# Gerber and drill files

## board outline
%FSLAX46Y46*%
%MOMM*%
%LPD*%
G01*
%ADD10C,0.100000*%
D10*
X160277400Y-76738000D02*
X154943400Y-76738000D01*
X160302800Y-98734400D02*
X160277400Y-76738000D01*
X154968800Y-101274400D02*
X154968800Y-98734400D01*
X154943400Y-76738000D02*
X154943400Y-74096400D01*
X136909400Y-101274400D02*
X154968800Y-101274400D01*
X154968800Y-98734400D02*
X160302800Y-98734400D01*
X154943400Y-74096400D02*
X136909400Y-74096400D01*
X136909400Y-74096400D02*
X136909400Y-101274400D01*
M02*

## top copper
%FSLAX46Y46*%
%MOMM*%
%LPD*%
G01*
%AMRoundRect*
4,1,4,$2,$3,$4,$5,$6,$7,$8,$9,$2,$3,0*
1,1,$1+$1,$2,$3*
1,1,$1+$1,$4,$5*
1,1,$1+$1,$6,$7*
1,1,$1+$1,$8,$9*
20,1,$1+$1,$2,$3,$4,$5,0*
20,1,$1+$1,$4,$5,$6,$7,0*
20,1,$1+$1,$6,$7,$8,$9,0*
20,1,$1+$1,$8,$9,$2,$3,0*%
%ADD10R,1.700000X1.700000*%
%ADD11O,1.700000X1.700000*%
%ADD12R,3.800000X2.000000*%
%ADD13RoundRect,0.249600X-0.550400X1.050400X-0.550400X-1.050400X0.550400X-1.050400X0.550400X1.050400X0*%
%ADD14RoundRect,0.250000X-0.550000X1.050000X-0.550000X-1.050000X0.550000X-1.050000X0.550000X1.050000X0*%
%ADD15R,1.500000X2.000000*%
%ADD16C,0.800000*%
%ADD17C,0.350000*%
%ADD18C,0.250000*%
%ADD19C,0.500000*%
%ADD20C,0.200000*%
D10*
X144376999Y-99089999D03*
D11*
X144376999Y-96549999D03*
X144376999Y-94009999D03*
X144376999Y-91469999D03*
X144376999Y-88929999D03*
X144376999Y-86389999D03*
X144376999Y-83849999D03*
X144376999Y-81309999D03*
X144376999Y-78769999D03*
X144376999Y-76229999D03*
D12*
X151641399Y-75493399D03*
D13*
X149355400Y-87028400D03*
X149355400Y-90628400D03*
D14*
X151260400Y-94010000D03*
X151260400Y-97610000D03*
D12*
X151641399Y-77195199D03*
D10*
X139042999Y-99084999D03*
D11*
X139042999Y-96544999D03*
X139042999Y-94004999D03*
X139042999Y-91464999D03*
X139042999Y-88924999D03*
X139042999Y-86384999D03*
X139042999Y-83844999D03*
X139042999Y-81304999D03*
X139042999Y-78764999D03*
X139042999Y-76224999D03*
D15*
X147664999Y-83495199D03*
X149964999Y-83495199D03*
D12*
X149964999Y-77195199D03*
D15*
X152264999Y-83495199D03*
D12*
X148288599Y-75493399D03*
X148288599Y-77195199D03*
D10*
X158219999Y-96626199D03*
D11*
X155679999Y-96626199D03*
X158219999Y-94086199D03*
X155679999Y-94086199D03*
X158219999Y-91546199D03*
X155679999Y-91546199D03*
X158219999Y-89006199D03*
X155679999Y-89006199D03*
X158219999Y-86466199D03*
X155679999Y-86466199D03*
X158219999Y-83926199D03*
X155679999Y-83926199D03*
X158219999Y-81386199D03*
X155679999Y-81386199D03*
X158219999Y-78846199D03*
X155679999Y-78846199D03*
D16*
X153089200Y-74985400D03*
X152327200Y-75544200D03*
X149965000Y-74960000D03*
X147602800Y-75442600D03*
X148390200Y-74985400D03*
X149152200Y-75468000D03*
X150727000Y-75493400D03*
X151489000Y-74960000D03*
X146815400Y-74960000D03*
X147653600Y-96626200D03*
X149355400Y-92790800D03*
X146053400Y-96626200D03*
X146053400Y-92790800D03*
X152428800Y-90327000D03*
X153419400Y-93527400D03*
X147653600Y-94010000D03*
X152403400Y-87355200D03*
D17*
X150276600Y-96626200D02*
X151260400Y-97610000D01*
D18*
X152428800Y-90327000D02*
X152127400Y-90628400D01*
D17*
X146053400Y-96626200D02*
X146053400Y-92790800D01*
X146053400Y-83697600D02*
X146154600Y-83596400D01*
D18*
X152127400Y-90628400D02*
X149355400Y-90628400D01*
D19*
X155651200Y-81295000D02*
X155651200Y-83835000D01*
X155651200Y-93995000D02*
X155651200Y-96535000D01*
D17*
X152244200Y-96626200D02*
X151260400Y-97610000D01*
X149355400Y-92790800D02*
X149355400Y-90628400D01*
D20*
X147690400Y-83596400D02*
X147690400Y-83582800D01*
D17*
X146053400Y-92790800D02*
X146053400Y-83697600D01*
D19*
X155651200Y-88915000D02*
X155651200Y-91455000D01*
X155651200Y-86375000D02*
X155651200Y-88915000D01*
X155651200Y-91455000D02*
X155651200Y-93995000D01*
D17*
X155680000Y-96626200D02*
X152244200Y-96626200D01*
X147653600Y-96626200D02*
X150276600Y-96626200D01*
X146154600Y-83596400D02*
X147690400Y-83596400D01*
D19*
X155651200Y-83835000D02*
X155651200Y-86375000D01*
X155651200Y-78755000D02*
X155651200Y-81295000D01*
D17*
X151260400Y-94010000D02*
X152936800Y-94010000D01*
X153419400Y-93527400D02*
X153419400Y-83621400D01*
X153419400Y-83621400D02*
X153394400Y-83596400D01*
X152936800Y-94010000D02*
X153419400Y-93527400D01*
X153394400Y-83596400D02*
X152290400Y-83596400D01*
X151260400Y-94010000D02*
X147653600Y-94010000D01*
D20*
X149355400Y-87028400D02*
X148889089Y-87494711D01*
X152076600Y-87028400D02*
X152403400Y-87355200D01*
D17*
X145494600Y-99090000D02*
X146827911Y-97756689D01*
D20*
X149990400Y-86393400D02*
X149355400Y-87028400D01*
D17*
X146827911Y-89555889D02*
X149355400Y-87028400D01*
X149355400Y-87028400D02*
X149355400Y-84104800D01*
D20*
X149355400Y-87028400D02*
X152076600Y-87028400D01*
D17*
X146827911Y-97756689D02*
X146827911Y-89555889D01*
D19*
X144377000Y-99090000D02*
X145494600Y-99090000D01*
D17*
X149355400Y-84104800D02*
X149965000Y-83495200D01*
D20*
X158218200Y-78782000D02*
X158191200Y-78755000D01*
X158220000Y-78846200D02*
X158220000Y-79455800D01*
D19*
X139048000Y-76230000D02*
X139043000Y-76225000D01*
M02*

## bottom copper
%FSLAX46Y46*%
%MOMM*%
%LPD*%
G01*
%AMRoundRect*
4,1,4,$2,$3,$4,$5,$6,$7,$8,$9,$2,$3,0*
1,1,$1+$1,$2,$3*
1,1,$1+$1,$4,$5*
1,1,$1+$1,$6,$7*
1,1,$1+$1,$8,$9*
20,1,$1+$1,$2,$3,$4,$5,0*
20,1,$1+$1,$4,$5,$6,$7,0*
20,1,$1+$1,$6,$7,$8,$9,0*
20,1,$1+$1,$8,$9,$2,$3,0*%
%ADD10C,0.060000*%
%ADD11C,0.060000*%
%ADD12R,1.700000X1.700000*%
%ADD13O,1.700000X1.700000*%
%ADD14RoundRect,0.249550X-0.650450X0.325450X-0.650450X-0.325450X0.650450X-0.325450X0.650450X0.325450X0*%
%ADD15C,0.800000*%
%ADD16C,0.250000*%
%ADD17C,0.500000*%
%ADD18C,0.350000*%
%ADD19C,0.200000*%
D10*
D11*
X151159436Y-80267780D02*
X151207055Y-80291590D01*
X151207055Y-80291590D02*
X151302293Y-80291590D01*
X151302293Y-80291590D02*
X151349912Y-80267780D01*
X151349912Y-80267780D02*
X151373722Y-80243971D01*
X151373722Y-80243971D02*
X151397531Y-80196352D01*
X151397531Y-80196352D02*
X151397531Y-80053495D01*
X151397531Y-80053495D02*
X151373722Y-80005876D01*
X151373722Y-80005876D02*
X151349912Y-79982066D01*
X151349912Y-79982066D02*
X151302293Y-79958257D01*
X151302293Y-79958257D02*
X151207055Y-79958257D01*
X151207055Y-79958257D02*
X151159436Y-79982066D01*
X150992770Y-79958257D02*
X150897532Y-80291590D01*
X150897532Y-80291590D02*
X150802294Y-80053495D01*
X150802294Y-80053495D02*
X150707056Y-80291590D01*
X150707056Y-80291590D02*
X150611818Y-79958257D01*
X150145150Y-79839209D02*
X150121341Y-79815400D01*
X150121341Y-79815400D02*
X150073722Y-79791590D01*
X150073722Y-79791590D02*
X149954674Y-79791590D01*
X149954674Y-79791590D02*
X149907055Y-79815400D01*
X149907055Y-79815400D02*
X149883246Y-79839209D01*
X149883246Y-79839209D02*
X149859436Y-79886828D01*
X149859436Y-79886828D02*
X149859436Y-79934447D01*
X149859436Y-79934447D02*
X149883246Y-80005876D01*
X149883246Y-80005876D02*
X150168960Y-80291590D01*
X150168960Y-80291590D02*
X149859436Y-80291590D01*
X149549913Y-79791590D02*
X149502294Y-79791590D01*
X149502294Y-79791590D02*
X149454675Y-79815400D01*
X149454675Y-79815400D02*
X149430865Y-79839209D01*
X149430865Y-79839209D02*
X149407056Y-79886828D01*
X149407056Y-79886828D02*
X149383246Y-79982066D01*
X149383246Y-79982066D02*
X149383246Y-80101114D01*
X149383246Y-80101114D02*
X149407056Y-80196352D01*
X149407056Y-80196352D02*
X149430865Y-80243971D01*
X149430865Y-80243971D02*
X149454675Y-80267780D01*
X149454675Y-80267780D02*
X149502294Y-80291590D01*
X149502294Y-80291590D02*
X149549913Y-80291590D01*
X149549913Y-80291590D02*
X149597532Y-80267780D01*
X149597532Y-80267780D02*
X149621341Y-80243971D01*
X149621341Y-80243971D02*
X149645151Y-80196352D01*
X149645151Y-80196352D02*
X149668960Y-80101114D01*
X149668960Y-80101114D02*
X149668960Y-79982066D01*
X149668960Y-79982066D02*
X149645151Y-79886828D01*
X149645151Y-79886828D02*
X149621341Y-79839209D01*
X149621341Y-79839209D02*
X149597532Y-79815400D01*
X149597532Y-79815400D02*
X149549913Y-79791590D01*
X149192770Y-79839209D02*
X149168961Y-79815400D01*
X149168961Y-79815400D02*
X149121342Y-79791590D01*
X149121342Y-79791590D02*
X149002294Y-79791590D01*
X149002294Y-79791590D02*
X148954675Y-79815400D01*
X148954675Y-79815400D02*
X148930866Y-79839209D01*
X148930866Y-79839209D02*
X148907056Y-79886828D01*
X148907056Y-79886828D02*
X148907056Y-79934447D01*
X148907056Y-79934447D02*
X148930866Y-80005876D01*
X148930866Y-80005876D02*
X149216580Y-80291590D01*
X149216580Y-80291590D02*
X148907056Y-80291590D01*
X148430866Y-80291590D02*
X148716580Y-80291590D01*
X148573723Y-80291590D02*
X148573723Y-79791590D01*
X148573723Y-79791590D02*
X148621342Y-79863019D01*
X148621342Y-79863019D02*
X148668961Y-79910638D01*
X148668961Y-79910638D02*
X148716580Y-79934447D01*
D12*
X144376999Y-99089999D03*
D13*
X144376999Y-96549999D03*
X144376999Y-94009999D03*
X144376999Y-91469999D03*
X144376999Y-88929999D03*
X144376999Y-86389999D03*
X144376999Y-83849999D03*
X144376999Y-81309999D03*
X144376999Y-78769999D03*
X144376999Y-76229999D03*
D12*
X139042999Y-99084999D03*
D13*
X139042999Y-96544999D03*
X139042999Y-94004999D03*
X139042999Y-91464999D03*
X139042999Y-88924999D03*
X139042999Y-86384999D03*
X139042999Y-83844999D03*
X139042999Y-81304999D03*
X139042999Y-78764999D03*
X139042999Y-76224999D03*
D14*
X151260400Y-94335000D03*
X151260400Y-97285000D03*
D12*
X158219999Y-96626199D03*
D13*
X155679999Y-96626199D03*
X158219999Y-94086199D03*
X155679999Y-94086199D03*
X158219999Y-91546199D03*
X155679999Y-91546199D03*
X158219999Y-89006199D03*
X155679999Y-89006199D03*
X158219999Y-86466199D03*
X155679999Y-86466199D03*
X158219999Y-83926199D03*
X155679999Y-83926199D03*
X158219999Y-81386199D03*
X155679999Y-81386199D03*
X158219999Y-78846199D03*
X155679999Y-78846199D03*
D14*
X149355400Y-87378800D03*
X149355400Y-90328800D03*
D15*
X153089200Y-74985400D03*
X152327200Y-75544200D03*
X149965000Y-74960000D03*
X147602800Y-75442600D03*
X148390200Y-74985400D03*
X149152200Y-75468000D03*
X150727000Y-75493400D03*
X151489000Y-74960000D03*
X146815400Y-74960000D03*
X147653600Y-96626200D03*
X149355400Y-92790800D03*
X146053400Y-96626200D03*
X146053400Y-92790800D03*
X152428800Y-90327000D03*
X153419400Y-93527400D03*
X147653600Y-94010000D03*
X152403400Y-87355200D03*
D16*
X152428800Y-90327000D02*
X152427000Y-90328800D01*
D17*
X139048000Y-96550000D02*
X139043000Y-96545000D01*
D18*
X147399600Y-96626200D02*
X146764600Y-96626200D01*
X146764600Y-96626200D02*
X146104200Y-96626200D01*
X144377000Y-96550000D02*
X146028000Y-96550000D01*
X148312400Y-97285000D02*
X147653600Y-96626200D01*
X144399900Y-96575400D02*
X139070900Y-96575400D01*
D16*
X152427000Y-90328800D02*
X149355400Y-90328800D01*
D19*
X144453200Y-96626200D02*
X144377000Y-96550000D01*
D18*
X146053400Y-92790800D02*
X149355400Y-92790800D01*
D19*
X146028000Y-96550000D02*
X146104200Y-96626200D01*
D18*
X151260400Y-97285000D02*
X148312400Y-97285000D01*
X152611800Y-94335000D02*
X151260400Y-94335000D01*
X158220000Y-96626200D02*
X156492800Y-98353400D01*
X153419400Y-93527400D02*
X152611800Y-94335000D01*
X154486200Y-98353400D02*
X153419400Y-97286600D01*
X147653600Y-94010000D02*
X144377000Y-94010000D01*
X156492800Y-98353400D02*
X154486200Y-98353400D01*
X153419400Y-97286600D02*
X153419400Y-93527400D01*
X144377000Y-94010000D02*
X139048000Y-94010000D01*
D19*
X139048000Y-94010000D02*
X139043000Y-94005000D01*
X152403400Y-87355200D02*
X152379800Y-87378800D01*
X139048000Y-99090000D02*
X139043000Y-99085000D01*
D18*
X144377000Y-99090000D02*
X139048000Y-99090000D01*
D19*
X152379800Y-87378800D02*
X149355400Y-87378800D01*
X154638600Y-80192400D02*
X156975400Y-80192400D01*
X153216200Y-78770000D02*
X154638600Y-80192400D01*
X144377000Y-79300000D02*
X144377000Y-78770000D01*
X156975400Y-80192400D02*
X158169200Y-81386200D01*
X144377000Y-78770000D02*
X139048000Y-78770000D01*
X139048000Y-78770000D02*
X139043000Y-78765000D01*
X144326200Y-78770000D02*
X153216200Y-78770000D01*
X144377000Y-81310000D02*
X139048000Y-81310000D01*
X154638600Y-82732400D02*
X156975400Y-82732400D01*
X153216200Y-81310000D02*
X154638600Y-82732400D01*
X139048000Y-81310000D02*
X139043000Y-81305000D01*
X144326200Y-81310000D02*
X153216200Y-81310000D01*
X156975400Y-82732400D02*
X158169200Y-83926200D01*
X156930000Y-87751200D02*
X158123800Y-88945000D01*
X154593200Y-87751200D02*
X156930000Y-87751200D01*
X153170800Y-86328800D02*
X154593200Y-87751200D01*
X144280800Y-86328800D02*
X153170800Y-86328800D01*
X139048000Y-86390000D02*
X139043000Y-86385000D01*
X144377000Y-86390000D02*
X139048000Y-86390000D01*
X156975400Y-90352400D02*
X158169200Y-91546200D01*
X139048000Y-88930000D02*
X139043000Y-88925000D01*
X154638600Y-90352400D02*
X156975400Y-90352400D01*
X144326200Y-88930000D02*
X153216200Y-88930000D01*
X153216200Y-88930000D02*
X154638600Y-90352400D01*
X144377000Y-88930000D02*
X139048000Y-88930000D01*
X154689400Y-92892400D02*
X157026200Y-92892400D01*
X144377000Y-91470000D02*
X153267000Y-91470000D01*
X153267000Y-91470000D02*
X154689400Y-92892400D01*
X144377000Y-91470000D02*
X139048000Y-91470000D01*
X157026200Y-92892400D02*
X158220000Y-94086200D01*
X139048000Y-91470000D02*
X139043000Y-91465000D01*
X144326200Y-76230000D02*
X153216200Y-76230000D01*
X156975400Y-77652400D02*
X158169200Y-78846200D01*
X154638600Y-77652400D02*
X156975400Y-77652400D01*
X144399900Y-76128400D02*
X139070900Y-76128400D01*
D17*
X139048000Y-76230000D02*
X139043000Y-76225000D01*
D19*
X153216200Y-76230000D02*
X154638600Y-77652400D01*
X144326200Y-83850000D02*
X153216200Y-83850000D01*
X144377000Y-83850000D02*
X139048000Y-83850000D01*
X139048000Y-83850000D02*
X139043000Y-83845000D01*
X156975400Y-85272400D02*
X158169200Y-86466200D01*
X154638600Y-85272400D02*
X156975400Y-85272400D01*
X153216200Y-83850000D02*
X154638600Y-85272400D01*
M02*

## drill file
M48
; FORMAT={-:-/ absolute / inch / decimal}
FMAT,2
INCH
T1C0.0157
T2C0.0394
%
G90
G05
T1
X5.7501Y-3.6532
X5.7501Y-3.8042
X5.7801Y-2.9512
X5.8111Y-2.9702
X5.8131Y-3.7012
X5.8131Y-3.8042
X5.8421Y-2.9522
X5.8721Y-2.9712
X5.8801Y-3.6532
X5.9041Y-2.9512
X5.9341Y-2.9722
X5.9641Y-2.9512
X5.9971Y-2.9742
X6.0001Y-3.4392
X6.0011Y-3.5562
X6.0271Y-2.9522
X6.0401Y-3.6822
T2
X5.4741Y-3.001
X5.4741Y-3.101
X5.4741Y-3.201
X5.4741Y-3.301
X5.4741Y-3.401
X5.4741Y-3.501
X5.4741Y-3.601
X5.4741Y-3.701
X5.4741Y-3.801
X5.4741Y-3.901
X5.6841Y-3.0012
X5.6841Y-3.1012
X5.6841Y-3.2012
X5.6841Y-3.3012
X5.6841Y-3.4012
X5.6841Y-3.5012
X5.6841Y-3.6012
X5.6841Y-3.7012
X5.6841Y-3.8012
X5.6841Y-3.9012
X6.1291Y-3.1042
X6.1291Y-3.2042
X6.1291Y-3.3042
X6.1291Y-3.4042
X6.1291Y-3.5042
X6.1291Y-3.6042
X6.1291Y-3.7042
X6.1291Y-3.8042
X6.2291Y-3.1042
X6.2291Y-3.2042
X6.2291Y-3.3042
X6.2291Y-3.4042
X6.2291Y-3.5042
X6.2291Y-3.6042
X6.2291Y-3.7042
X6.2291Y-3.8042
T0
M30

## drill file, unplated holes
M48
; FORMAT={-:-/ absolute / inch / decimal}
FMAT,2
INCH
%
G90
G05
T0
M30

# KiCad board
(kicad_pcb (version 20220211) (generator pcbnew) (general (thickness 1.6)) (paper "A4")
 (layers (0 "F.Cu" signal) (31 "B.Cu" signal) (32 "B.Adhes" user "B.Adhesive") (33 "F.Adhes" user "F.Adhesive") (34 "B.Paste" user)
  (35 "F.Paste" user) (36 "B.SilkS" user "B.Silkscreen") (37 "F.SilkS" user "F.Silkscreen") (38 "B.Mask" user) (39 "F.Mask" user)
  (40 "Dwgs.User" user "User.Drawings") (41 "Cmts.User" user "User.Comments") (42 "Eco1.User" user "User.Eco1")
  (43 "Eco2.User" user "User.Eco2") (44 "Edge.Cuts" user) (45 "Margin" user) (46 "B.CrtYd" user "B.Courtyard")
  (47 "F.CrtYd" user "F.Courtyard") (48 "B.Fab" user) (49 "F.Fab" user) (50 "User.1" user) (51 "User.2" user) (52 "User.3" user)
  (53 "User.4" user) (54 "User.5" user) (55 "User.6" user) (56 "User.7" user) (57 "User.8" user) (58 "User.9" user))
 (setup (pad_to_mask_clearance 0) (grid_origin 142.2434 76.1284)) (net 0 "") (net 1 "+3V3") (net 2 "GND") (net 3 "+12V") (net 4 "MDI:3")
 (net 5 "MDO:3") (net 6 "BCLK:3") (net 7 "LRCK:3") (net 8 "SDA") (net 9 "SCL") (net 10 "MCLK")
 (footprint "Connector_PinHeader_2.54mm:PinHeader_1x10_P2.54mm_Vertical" (layer "F.Cu") (at 144.377 99.09 180)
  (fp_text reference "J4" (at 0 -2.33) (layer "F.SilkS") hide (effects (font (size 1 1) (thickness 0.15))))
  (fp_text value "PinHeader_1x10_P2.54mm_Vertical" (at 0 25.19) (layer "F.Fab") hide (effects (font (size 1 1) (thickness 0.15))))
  (pad "0" thru_hole rect locked (at 0 0 180) (size 1.7 1.7) (drill 1) (layers *.Cu *.Mask) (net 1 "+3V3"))
  (pad "1" thru_hole oval locked (at 0 2.54 180) (size 1.7 1.7) (drill 1) (layers *.Cu *.Mask) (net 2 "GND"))
  (pad "2" thru_hole oval locked (at 0 5.08 180) (size 1.7 1.7) (drill 1) (layers *.Cu *.Mask) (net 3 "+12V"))
  (pad "3" thru_hole oval locked (at 0 7.62 180) (size 1.7 1.7) (drill 1) (layers *.Cu *.Mask) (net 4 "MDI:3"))
  (pad "4" thru_hole oval locked (at 0 10.16 180) (size 1.7 1.7) (drill 1) (layers *.Cu *.Mask) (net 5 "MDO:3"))
  (pad "5" thru_hole oval locked (at 0 12.7 180) (size 1.7 1.7) (drill 1) (layers *.Cu *.Mask) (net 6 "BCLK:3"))
  (pad "6" thru_hole oval locked (at 0 15.24 180) (size 1.7 1.7) (drill 1) (layers *.Cu *.Mask) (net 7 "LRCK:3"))
  (pad "7" thru_hole oval locked (at 0 17.78 180) (size 1.7 1.7) (drill 1) (layers *.Cu *.Mask) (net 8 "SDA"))
  (pad "8" thru_hole oval locked (at 0 20.32 180) (size 1.7 1.7) (drill 1) (layers *.Cu *.Mask) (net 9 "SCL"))
  (pad "9" thru_hole oval locked (at 0 22.86 180) (size 1.7 1.7) (drill 1) (layers *.Cu *.Mask) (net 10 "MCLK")))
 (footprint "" (layer "F.Cu") (at 151.6414 75.4934)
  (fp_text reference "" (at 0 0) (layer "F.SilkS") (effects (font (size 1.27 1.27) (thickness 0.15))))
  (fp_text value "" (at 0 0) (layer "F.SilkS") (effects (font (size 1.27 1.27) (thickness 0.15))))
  (pad "2" smd rect locked (at 0 0 90) (size 2 3.8) (layers "F.Cu" "F.Paste" "F.Mask")))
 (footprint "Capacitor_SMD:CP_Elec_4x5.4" (layer "F.Cu") (at 149.3554 88.8284 -90)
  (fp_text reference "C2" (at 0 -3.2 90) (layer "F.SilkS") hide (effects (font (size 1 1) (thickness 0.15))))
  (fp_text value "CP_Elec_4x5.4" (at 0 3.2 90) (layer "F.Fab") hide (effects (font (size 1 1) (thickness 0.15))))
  (pad "1" smd roundrect locked (at -1.8 0 270) (size 2.6 1.6) (layers "F.Cu" "F.Paste" "F.Mask") (roundrect_rratio 0.156) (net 1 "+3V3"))
  (pad "2" smd roundrect locked (at 1.8 0 270) (size 2.6 1.6) (layers "F.Cu" "F.Paste" "F.Mask") (roundrect_rratio 0.156) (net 2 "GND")))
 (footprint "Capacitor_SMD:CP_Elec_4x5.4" (layer "F.Cu") (at 151.2604 95.81 -90)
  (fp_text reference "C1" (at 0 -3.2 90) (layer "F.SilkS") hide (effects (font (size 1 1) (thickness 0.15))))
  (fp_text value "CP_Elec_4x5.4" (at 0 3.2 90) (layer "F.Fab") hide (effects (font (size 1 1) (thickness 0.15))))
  (pad "1" smd roundrect locked (at -1.8 0 270) (size 2.6 1.6) (layers "F.Cu" "F.Paste" "F.Mask") (roundrect_rratio 0.15625) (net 3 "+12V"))
  (pad "2" smd roundrect locked (at 1.8 0 270) (size 2.6 1.6) (layers "F.Cu" "F.Paste" "F.Mask") (roundrect_rratio 0.15625) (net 2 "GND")))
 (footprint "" (layer "F.Cu") (at 151.6414 77.1952)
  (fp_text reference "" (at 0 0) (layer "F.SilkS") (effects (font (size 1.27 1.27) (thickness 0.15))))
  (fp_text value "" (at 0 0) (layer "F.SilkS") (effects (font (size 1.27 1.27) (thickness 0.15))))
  (pad "2" smd rect locked (at 0 0 90) (size 2 3.8) (layers "F.Cu" "F.Paste" "F.Mask")))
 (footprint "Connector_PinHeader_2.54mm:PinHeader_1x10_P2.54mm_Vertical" (layer "F.Cu") (at 139.043 99.085 180)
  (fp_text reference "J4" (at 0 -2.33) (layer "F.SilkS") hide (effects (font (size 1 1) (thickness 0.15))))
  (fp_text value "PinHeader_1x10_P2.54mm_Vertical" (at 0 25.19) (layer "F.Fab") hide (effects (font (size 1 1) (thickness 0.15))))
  (pad "0" thru_hole rect locked (at 0 0 180) (size 1.7 1.7) (drill 1) (layers *.Cu *.Mask) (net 1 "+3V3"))
  (pad "1" thru_hole oval locked (at 0 2.54 180) (size 1.7 1.7) (drill 1) (layers *.Cu *.Mask) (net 2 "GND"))
  (pad "2" thru_hole oval locked (at 0 5.08 180) (size 1.7 1.7) (drill 1) (layers *.Cu *.Mask) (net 3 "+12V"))
  (pad "3" thru_hole oval locked (at 0 7.62 180) (size 1.7 1.7) (drill 1) (layers *.Cu *.Mask) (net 4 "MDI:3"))
  (pad "4" thru_hole oval locked (at 0 10.16 180) (size 1.7 1.7) (drill 1) (layers *.Cu *.Mask) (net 5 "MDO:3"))
  (pad "5" thru_hole oval locked (at 0 12.7 180) (size 1.7 1.7) (drill 1) (layers *.Cu *.Mask) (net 6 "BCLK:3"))
  (pad "6" thru_hole oval locked (at 0 15.24 180) (size 1.7 1.7) (drill 1) (layers *.Cu *.Mask) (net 7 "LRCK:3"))
  (pad "7" thru_hole oval locked (at 0 17.78 180) (size 1.7 1.7) (drill 1) (layers *.Cu *.Mask) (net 8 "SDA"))
  (pad "8" thru_hole oval locked (at 0 20.32 180) (size 1.7 1.7) (drill 1) (layers *.Cu *.Mask) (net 9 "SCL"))
  (pad "9" thru_hole oval locked (at 0 22.86 180) (size 1.7 1.7) (drill 1) (layers *.Cu *.Mask) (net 10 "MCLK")))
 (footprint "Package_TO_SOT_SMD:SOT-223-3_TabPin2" (layer "F.Cu") (at 149.965 80.3452 90)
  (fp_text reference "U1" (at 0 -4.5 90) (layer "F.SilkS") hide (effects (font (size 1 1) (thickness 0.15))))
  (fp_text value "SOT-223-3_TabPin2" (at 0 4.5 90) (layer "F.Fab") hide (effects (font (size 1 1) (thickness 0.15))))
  (pad "1" smd rect locked (at -3.15 -2.3 90) (size 2 1.5) (layers "F.Cu" "F.Paste" "F.Mask") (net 2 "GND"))
  (pad "2" smd rect locked (at -3.15 0 90) (size 2 1.5) (layers "F.Cu" "F.Paste" "F.Mask") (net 1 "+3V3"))
  (pad "2" smd rect locked (at 3.15 0 90) (size 2 3.8) (layers "F.Cu" "F.Paste" "F.Mask"))
  (pad "3" smd rect locked (at -3.15 2.3 90) (size 2 1.5) (layers "F.Cu" "F.Paste" "F.Mask") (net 3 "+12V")))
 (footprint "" (layer "F.Cu") (at 148.2886 75.4934)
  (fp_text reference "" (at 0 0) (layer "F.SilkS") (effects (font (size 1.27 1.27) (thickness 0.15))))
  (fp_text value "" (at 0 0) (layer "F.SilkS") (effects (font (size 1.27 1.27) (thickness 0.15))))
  (pad "2" smd rect locked (at 0 0 90) (size 2 3.8) (layers "F.Cu" "F.Paste" "F.Mask")))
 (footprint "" (layer "F.Cu") (at 148.2886 77.1952)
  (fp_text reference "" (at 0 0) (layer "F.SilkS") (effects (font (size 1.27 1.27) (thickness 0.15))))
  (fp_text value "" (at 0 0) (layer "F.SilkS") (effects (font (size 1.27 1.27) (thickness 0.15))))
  (pad "2" smd rect locked (at 0 0 90) (size 2 3.8) (layers "F.Cu" "F.Paste" "F.Mask")))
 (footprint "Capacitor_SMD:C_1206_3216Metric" (layer "B.Cu") (at 151.2604 95.81 -90)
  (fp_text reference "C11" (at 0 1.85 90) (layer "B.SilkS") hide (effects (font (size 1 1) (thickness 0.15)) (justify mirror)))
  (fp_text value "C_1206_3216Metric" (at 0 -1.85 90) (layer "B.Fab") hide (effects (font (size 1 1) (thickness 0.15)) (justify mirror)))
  (pad "1" smd roundrect locked (at -1.475 0 270) (size 1.15 1.8) (layers "B.Cu" "B.Paste" "B.Mask") (roundrect_rratio 0.217) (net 3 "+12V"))
  (pad "2" smd roundrect locked (at 1.475 0 270) (size 1.15 1.8) (layers "B.Cu" "B.Paste" "B.Mask") (roundrect_rratio 0.217) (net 2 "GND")))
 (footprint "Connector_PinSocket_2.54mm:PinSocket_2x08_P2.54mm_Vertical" (layer "B.Cu") (at 158.22 96.6262)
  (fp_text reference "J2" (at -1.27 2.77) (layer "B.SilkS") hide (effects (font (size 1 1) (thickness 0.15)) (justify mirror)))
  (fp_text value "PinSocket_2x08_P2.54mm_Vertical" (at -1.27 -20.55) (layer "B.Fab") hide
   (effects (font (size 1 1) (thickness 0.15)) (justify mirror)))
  (pad "1" thru_hole rect locked (at 0 0) (size 1.7 1.7) (drill 1) (layers *.Cu *.Mask) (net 3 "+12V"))
  (pad "2" thru_hole oval locked (at -2.54 0) (size 1.7 1.7) (drill 1) (layers *.Cu *.Mask) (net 2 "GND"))
  (pad "3" thru_hole oval locked (at 0 -2.54) (size 1.7 1.7) (drill 1) (layers *.Cu *.Mask) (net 4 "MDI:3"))
  (pad "4" thru_hole oval locked (at -2.54 -2.54) (size 1.7 1.7) (drill 1) (layers *.Cu *.Mask) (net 2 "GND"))
  (pad "5" thru_hole oval locked (at 0 -5.08) (size 1.7 1.7) (drill 1) (layers *.Cu *.Mask) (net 5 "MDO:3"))
  (pad "6" thru_hole oval locked (at -2.54 -5.08) (size 1.7 1.7) (drill 1) (layers *.Cu *.Mask) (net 2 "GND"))
  (pad "7" thru_hole oval locked (at 0 -7.62) (size 1.7 1.7) (drill 1) (layers *.Cu *.Mask) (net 6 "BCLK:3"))
  (pad "8" thru_hole oval locked (at -2.54 -7.62) (size 1.7 1.7) (drill 1) (layers *.Cu *.Mask) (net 2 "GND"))
  (pad "9" thru_hole oval locked (at 0 -10.16) (size 1.7 1.7) (drill 1) (layers *.Cu *.Mask) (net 7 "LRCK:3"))
  (pad "10" thru_hole oval locked (at -2.54 -10.16) (size 1.7 1.7) (drill 1) (layers *.Cu *.Mask) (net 2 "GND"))
  (pad "11" thru_hole oval locked (at 0 -12.7) (size 1.7 1.7) (drill 1) (layers *.Cu *.Mask) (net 8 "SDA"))
  (pad "12" thru_hole oval locked (at -2.54 -12.7) (size 1.7 1.7) (drill 1) (layers *.Cu *.Mask) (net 2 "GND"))
  (pad "13" thru_hole oval locked (at 0 -15.24) (size 1.7 1.7) (drill 1) (layers *.Cu *.Mask) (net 9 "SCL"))
  (pad "14" thru_hole oval locked (at -2.54 -15.24) (size 1.7 1.7) (drill 1) (layers *.Cu *.Mask) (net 2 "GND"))
  (pad "15" thru_hole oval locked (at 0 -17.78) (size 1.7 1.7) (drill 1) (layers *.Cu *.Mask) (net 10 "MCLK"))
  (pad "16" thru_hole oval locked (at -2.54 -17.78) (size 1.7 1.7) (drill 1) (layers *.Cu *.Mask) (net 2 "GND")))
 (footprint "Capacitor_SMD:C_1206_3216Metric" (layer "B.Cu") (at 149.3554 88.8538 -90)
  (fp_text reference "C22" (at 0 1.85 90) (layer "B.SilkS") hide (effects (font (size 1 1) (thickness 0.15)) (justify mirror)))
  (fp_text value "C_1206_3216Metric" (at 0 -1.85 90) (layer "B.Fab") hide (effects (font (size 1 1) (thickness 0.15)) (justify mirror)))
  (pad "1" smd roundrect locked (at -1.475 0 270) (size 1.15 1.8) (layers "B.Cu" "B.Paste" "B.Mask") (roundrect_rratio 0.217) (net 1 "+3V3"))
  (pad "2" smd roundrect locked (at 1.475 0 270) (size 1.15 1.8) (layers "B.Cu" "B.Paste" "B.Mask") (roundrect_rratio 0.217) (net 2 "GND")))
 (gr_line (start 160.2774 76.738) (end 154.9434 76.738) (stroke (width 0.1) (type solid)) (layer "Edge.Cuts"))
 (gr_line (start 160.3028 98.7344) (end 160.2774 76.738) (stroke (width 0.1) (type solid)) (layer "Edge.Cuts"))
 (gr_line (start 154.9688 101.2744) (end 154.9688 98.7344) (stroke (width 0.1) (type solid)) (layer "Edge.Cuts"))
 (gr_line (start 154.9434 76.738) (end 154.9434 74.0964) (stroke (width 0.1) (type solid)) (layer "Edge.Cuts"))
 (gr_line (start 136.9094 101.2744) (end 154.9688 101.2744) (stroke (width 0.1) (type solid)) (layer "Edge.Cuts"))
 (gr_line (start 154.9688 98.7344) (end 160.3028 98.7344) (stroke (width 0.1) (type solid)) (layer "Edge.Cuts"))
 (gr_line (start 154.9434 74.0964) (end 136.9094 74.0964) (stroke (width 0.1) (type solid)) (layer "Edge.Cuts"))
 (gr_line (start 136.9094 74.0964) (end 136.9094 101.2744) (stroke (width 0.1) (type solid)) (layer "Edge.Cuts"))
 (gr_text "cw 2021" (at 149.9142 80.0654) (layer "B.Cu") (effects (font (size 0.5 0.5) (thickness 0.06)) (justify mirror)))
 (via (at 153.0892 74.9854) (size 0.8) (drill 0.4) (layers "F.Cu" "B.Cu") (free) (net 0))
 (via (at 152.3272 75.5442) (size 0.8) (drill 0.4) (layers "F.Cu" "B.Cu") (free) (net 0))
 (via (at 149.965 74.96) (size 0.8) (drill 0.4) (layers "F.Cu" "B.Cu") (free) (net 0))
 (via (at 147.6028 75.4426) (size 0.8) (drill 0.4) (layers "F.Cu" "B.Cu") (free) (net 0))
 (via (at 148.3902 74.9854) (size 0.8) (drill 0.4) (layers "F.Cu" "B.Cu") (free) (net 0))
 (via (at 149.1522 75.468) (size 0.8) (drill 0.4) (layers "F.Cu" "B.Cu") (free) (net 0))
 (via (at 150.727 75.4934) (size 0.8) (drill 0.4) (layers "F.Cu" "B.Cu") (free) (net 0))
 (via (at 151.489 74.96) (size 0.8) (drill 0.4) (layers "F.Cu" "B.Cu") (free) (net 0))
 (via (at 146.8154 74.96) (size 0.8) (drill 0.4) (layers "F.Cu" "B.Cu") (free) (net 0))
 (segment (start 150.2766 96.6262) (end 151.2604 97.61) (width 0.35) (layer "F.Cu") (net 2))
 (segment (start 152.4288 90.327) (end 152.1274 90.6284) (width 0.25) (layer "F.Cu") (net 2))
 (segment (start 146.0534 96.6262) (end 146.0534 92.7908) (width 0.35) (layer "F.Cu") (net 2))
 (segment (start 146.0534 83.6976) (end 146.1546 83.5964) (width 0.35) (layer "F.Cu") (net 2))
 (segment (start 152.1274 90.6284) (end 149.3554 90.6284) (width 0.25) (layer "F.Cu") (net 2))
 (segment (start 155.6512 81.295) (end 155.6512 83.835) (width 0.5) (layer "F.Cu") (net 2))
 (segment (start 155.6512 93.995) (end 155.6512 96.535) (width 0.5) (layer "F.Cu") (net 2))
 (segment (start 152.2442 96.6262) (end 151.2604 97.61) (width 0.35) (layer "F.Cu") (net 2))
 (segment (start 149.3554 92.7908) (end 149.3554 90.6284) (width 0.35) (layer "F.Cu") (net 2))
 (segment (start 147.6904 83.5964) (end 147.6904 83.5828) (width 0.2) (layer "F.Cu") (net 2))
 (segment (start 146.0534 92.7908) (end 146.0534 83.6976) (width 0.35) (layer "F.Cu") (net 2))
 (segment (start 155.6512 88.915) (end 155.6512 91.455) (width 0.5) (layer "F.Cu") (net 2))
 (segment (start 155.6512 86.375) (end 155.6512 88.915) (width 0.5) (layer "F.Cu") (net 2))
 (segment (start 155.6512 91.455) (end 155.6512 93.995) (width 0.5) (layer "F.Cu") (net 2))
 (segment (start 155.68 96.6262) (end 152.2442 96.6262) (width 0.35) (layer "F.Cu") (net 2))
 (segment (start 147.6536 96.6262) (end 150.2766 96.6262) (width 0.35) (layer "F.Cu") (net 2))
 (segment (start 146.1546 83.5964) (end 147.6904 83.5964) (width 0.35) (layer "F.Cu") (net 2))
 (segment (start 155.6512 83.835) (end 155.6512 86.375) (width 0.5) (layer "F.Cu") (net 2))
 (segment (start 155.6512 78.755) (end 155.6512 81.295) (width 0.5) (layer "F.Cu") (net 2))
 (via (at 147.6536 96.6262) (size 0.8) (drill 0.4) (layers "F.Cu" "B.Cu") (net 2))
 (via (at 149.3554 92.7908) (size 0.8) (drill 0.4) (layers "F.Cu" "B.Cu") (free) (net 2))
 (via (at 146.0534 96.6262) (size 0.8) (drill 0.4) (layers "F.Cu" "B.Cu") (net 2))
 (via (at 146.0534 92.7908) (size 0.8) (drill 0.4) (layers "F.Cu" "B.Cu") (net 2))
 (via (at 152.4288 90.327) (size 0.8) (drill 0.4) (layers "F.Cu" "B.Cu") (free) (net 2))
 (segment (start 152.4288 90.327) (end 152.427 90.3288) (width 0.25) (layer "B.Cu") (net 2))
 (segment (start 139.048 96.55) (end 139.043 96.545) (width 0.5) (layer "B.Cu") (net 2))
 (segment (start 147.3996 96.6262) (end 146.7646 96.6262) (width 0.35) (layer "B.Cu") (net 2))
 (segment (start 146.7646 96.6262) (end 146.1042 96.6262) (width 0.35) (layer "B.Cu") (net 2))
 (segment (start 144.377 96.55) (end 146.028 96.55) (width 0.35) (layer "B.Cu") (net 2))
 (segment (start 148.3124 97.285) (end 147.6536 96.6262) (width 0.35) (layer "B.Cu") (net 2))
 (segment (start 144.3999 96.5754) (end 139.0709 96.5754) (width 0.35) (layer "B.Cu") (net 2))
 (segment (start 152.427 90.3288) (end 149.3554 90.3288) (width 0.25) (layer "B.Cu") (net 2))
 (segment (start 144.4532 96.6262) (end 144.377 96.55) (width 0.2) (layer "B.Cu") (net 2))
 (segment (start 146.0534 92.7908) (end 149.3554 92.7908) (width 0.35) (layer "B.Cu") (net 2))
 (segment (start 146.028 96.55) (end 146.1042 96.6262) (width 0.2) (layer "B.Cu") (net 2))
 (segment (start 151.2604 97.285) (end 148.3124 97.285) (width 0.35) (layer "B.Cu") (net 2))
 (segment (start 151.2604 94.01) (end 152.9368 94.01) (width 0.35) (layer "F.Cu") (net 3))
 (segment (start 153.4194 93.5274) (end 153.4194 83.6214) (width 0.35) (layer "F.Cu") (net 3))
 (segment (start 153.4194 83.6214) (end 153.3944 83.5964) (width 0.35) (layer "F.Cu") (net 3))
 (segment (start 152.9368 94.01) (end 153.4194 93.5274) (width 0.35) (layer "F.Cu") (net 3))
 (segment (start 153.3944 83.5964) (end 152.2904 83.5964) (width 0.35) (layer "F.Cu") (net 3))
 (segment (start 151.2604 94.01) (end 147.6536 94.01) (width 0.35) (layer "F.Cu") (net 3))
 (via (at 153.4194 93.5274) (size 0.8) (drill 0.4) (layers "F.Cu" "B.Cu") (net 3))
 (via (at 147.6536 94.01) (size 0.8) (drill 0.4) (layers "F.Cu" "B.Cu") (free) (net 3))
 (segment (start 152.6118 94.335) (end 151.2604 94.335) (width 0.35) (layer "B.Cu") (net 3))
 (segment (start 158.22 96.6262) (end 156.4928 98.3534) (width 0.35) (layer "B.Cu") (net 3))
 (segment (start 153.4194 93.5274) (end 152.6118 94.335) (width 0.35) (layer "B.Cu") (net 3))
 (segment (start 154.4862 98.3534) (end 153.4194 97.2866) (width 0.35) (layer "B.Cu") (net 3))
 (segment (start 147.6536 94.01) (end 144.377 94.01) (width 0.35) (layer "B.Cu") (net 3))
 (segment (start 156.4928 98.3534) (end 154.4862 98.3534) (width 0.35) (layer "B.Cu") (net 3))
 (segment (start 153.4194 97.2866) (end 153.4194 93.5274) (width 0.35) (layer "B.Cu") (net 3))
 (segment (start 144.377 94.01) (end 139.048 94.01) (width 0.35) (layer "B.Cu") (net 3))
 (segment (start 139.048 94.01) (end 139.043 94.005) (width 0.2) (layer "B.Cu") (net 3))
 (segment (start 149.3554 87.0284) (end 148.889089 87.494711) (width 0.2) (layer "F.Cu") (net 1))
 (segment (start 152.0766 87.0284) (end 152.4034 87.3552) (width 0.2) (layer "F.Cu") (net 1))
 (segment (start 145.4946 99.09) (end 146.827911 97.756689) (width 0.35) (layer "F.Cu") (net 1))
 (segment (start 149.9904 86.3934) (end 149.3554 87.0284) (width 0.2) (layer "F.Cu") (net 1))
 (segment (start 146.827911 89.555889) (end 149.3554 87.0284) (width 0.35) (layer "F.Cu") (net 1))
 (segment (start 149.3554 87.0284) (end 149.3554 84.1048) (width 0.35) (layer "F.Cu") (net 1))
 (segment (start 149.3554 87.0284) (end 152.0766 87.0284) (width 0.2) (layer "F.Cu") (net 1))
 (segment (start 146.827911 97.756689) (end 146.827911 89.555889) (width 0.35) (layer "F.Cu") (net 1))
 (segment (start 144.377 99.09) (end 145.4946 99.09) (width 0.5) (layer "F.Cu") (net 1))
 (segment (start 149.3554 84.1048) (end 149.965 83.4952) (width 0.35) (layer "F.Cu") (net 1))
 (via (at 152.4034 87.3552) (size 0.8) (drill 0.4) (layers "F.Cu" "B.Cu") (free) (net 1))
 (segment (start 152.4034 87.3552) (end 152.3798 87.3788) (width 0.2) (layer "B.Cu") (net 1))
 (segment (start 139.048 99.09) (end 139.043 99.085) (width 0.2) (layer "B.Cu") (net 1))
 (segment (start 144.377 99.09) (end 139.048 99.09) (width 0.35) (layer "B.Cu") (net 1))
 (segment (start 152.3798 87.3788) (end 149.3554 87.3788) (width 0.2) (layer "B.Cu") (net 1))
 (segment (start 154.6386 80.1924) (end 156.9754 80.1924) (width 0.2) (layer "B.Cu") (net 9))
 (segment (start 153.2162 78.77) (end 154.6386 80.1924) (width 0.2) (layer "B.Cu") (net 9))
 (segment (start 144.377 79.3) (end 144.377 78.77) (width 0.2) (layer "B.Cu") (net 9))
 (segment (start 156.9754 80.1924) (end 158.1692 81.3862) (width 0.2) (layer "B.Cu") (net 9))
 (segment (start 144.377 78.77) (end 139.048 78.77) (width 0.2) (layer "B.Cu") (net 9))
 (segment (start 139.048 78.77) (end 139.043 78.765) (width 0.2) (layer "B.Cu") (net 9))
 (segment (start 144.3262 78.77) (end 153.2162 78.77) (width 0.2) (layer "B.Cu") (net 9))
 (segment (start 144.377 81.31) (end 139.048 81.31) (width 0.2) (layer "B.Cu") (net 8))
 (segment (start 154.6386 82.7324) (end 156.9754 82.7324) (width 0.2) (layer "B.Cu") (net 8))
 (segment (start 153.2162 81.31) (end 154.6386 82.7324) (width 0.2) (layer "B.Cu") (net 8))
 (segment (start 139.048 81.31) (end 139.043 81.305) (width 0.2) (layer "B.Cu") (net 8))
 (segment (start 144.3262 81.31) (end 153.2162 81.31) (width 0.2) (layer "B.Cu") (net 8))
 (segment (start 156.9754 82.7324) (end 158.1692 83.9262) (width 0.2) (layer "B.Cu") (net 8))
 (segment (start 156.93 87.7512) (end 158.1238 88.945) (width 0.2) (layer "B.Cu") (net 6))
 (segment (start 154.5932 87.7512) (end 156.93 87.7512) (width 0.2) (layer "B.Cu") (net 6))
 (segment (start 153.1708 86.3288) (end 154.5932 87.7512) (width 0.2) (layer "B.Cu") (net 6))
 (segment (start 144.2808 86.3288) (end 153.1708 86.3288) (width 0.2) (layer "B.Cu") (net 6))
 (segment (start 139.048 86.39) (end 139.043 86.385) (width 0.2) (layer "B.Cu") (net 6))
 (segment (start 144.377 86.39) (end 139.048 86.39) (width 0.2) (layer "B.Cu") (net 6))
 (segment (start 156.9754 90.3524) (end 158.1692 91.5462) (width 0.2) (layer "B.Cu") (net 5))
 (segment (start 139.048 88.93) (end 139.043 88.925) (width 0.2) (layer "B.Cu") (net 5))
 (segment (start 154.6386 90.3524) (end 156.9754 90.3524) (width 0.2) (layer "B.Cu") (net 5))
 (segment (start 144.3262 88.93) (end 153.2162 88.93) (width 0.2) (layer "B.Cu") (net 5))
 (segment (start 153.2162 88.93) (end 154.6386 90.3524) (width 0.2) (layer "B.Cu") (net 5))
 (segment (start 144.377 88.93) (end 139.048 88.93) (width 0.2) (layer "B.Cu") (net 5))
 (segment (start 154.6894 92.8924) (end 157.0262 92.8924) (width 0.2) (layer "B.Cu") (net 4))
 (segment (start 144.377 91.47) (end 153.267 91.47) (width 0.2) (layer "B.Cu") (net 4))
 (segment (start 153.267 91.47) (end 154.6894 92.8924) (width 0.2) (layer "B.Cu") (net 4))
 (segment (start 144.377 91.47) (end 139.048 91.47) (width 0.2) (layer "B.Cu") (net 4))
 (segment (start 157.0262 92.8924) (end 158.22 94.0862) (width 0.2) (layer "B.Cu") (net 4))
 (segment (start 139.048 91.47) (end 139.043 91.465) (width 0.2) (layer "B.Cu") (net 4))
 (segment (start 158.2182 78.782) (end 158.1912 78.755) (width 0.2) (layer "F.Cu") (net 10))
 (segment (start 158.22 78.8462) (end 158.22 79.4558) (width 0.2) (layer "F.Cu") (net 10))
 (segment (start 139.048 76.23) (end 139.043 76.225) (width 0.5) (layer "F.Cu") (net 10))
 (segment (start 144.3262 76.23) (end 153.2162 76.23) (width 0.2) (layer "B.Cu") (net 10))
 (segment (start 156.9754 77.6524) (end 158.1692 78.8462) (width 0.2) (layer "B.Cu") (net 10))
 (segment (start 154.6386 77.6524) (end 156.9754 77.6524) (width 0.2) (layer "B.Cu") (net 10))
 (segment (start 144.3999 76.1284) (end 139.0709 76.1284) (width 0.2) (layer "B.Cu") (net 10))
 (segment (start 139.048 76.23) (end 139.043 76.225) (width 0.5) (layer "B.Cu") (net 10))
 (segment (start 153.2162 76.23) (end 154.6386 77.6524) (width 0.2) (layer "B.Cu") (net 10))
 (segment (start 144.3262 83.85) (end 153.2162 83.85) (width 0.2) (layer "B.Cu") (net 7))
 (segment (start 144.377 83.85) (end 139.048 83.85) (width 0.2) (layer "B.Cu") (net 7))
 (segment (start 139.048 83.85) (end 139.043 83.845) (width 0.2) (layer "B.Cu") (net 7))
 (segment (start 156.9754 85.2724) (end 158.1692 86.4662) (width 0.2) (layer "B.Cu") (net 7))
 (segment (start 154.6386 85.2724) (end 156.9754 85.2724) (width 0.2) (layer "B.Cu") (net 7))
 (segment (start 153.2162 83.85) (end 154.6386 85.2724) (width 0.2) (layer "B.Cu") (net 7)))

